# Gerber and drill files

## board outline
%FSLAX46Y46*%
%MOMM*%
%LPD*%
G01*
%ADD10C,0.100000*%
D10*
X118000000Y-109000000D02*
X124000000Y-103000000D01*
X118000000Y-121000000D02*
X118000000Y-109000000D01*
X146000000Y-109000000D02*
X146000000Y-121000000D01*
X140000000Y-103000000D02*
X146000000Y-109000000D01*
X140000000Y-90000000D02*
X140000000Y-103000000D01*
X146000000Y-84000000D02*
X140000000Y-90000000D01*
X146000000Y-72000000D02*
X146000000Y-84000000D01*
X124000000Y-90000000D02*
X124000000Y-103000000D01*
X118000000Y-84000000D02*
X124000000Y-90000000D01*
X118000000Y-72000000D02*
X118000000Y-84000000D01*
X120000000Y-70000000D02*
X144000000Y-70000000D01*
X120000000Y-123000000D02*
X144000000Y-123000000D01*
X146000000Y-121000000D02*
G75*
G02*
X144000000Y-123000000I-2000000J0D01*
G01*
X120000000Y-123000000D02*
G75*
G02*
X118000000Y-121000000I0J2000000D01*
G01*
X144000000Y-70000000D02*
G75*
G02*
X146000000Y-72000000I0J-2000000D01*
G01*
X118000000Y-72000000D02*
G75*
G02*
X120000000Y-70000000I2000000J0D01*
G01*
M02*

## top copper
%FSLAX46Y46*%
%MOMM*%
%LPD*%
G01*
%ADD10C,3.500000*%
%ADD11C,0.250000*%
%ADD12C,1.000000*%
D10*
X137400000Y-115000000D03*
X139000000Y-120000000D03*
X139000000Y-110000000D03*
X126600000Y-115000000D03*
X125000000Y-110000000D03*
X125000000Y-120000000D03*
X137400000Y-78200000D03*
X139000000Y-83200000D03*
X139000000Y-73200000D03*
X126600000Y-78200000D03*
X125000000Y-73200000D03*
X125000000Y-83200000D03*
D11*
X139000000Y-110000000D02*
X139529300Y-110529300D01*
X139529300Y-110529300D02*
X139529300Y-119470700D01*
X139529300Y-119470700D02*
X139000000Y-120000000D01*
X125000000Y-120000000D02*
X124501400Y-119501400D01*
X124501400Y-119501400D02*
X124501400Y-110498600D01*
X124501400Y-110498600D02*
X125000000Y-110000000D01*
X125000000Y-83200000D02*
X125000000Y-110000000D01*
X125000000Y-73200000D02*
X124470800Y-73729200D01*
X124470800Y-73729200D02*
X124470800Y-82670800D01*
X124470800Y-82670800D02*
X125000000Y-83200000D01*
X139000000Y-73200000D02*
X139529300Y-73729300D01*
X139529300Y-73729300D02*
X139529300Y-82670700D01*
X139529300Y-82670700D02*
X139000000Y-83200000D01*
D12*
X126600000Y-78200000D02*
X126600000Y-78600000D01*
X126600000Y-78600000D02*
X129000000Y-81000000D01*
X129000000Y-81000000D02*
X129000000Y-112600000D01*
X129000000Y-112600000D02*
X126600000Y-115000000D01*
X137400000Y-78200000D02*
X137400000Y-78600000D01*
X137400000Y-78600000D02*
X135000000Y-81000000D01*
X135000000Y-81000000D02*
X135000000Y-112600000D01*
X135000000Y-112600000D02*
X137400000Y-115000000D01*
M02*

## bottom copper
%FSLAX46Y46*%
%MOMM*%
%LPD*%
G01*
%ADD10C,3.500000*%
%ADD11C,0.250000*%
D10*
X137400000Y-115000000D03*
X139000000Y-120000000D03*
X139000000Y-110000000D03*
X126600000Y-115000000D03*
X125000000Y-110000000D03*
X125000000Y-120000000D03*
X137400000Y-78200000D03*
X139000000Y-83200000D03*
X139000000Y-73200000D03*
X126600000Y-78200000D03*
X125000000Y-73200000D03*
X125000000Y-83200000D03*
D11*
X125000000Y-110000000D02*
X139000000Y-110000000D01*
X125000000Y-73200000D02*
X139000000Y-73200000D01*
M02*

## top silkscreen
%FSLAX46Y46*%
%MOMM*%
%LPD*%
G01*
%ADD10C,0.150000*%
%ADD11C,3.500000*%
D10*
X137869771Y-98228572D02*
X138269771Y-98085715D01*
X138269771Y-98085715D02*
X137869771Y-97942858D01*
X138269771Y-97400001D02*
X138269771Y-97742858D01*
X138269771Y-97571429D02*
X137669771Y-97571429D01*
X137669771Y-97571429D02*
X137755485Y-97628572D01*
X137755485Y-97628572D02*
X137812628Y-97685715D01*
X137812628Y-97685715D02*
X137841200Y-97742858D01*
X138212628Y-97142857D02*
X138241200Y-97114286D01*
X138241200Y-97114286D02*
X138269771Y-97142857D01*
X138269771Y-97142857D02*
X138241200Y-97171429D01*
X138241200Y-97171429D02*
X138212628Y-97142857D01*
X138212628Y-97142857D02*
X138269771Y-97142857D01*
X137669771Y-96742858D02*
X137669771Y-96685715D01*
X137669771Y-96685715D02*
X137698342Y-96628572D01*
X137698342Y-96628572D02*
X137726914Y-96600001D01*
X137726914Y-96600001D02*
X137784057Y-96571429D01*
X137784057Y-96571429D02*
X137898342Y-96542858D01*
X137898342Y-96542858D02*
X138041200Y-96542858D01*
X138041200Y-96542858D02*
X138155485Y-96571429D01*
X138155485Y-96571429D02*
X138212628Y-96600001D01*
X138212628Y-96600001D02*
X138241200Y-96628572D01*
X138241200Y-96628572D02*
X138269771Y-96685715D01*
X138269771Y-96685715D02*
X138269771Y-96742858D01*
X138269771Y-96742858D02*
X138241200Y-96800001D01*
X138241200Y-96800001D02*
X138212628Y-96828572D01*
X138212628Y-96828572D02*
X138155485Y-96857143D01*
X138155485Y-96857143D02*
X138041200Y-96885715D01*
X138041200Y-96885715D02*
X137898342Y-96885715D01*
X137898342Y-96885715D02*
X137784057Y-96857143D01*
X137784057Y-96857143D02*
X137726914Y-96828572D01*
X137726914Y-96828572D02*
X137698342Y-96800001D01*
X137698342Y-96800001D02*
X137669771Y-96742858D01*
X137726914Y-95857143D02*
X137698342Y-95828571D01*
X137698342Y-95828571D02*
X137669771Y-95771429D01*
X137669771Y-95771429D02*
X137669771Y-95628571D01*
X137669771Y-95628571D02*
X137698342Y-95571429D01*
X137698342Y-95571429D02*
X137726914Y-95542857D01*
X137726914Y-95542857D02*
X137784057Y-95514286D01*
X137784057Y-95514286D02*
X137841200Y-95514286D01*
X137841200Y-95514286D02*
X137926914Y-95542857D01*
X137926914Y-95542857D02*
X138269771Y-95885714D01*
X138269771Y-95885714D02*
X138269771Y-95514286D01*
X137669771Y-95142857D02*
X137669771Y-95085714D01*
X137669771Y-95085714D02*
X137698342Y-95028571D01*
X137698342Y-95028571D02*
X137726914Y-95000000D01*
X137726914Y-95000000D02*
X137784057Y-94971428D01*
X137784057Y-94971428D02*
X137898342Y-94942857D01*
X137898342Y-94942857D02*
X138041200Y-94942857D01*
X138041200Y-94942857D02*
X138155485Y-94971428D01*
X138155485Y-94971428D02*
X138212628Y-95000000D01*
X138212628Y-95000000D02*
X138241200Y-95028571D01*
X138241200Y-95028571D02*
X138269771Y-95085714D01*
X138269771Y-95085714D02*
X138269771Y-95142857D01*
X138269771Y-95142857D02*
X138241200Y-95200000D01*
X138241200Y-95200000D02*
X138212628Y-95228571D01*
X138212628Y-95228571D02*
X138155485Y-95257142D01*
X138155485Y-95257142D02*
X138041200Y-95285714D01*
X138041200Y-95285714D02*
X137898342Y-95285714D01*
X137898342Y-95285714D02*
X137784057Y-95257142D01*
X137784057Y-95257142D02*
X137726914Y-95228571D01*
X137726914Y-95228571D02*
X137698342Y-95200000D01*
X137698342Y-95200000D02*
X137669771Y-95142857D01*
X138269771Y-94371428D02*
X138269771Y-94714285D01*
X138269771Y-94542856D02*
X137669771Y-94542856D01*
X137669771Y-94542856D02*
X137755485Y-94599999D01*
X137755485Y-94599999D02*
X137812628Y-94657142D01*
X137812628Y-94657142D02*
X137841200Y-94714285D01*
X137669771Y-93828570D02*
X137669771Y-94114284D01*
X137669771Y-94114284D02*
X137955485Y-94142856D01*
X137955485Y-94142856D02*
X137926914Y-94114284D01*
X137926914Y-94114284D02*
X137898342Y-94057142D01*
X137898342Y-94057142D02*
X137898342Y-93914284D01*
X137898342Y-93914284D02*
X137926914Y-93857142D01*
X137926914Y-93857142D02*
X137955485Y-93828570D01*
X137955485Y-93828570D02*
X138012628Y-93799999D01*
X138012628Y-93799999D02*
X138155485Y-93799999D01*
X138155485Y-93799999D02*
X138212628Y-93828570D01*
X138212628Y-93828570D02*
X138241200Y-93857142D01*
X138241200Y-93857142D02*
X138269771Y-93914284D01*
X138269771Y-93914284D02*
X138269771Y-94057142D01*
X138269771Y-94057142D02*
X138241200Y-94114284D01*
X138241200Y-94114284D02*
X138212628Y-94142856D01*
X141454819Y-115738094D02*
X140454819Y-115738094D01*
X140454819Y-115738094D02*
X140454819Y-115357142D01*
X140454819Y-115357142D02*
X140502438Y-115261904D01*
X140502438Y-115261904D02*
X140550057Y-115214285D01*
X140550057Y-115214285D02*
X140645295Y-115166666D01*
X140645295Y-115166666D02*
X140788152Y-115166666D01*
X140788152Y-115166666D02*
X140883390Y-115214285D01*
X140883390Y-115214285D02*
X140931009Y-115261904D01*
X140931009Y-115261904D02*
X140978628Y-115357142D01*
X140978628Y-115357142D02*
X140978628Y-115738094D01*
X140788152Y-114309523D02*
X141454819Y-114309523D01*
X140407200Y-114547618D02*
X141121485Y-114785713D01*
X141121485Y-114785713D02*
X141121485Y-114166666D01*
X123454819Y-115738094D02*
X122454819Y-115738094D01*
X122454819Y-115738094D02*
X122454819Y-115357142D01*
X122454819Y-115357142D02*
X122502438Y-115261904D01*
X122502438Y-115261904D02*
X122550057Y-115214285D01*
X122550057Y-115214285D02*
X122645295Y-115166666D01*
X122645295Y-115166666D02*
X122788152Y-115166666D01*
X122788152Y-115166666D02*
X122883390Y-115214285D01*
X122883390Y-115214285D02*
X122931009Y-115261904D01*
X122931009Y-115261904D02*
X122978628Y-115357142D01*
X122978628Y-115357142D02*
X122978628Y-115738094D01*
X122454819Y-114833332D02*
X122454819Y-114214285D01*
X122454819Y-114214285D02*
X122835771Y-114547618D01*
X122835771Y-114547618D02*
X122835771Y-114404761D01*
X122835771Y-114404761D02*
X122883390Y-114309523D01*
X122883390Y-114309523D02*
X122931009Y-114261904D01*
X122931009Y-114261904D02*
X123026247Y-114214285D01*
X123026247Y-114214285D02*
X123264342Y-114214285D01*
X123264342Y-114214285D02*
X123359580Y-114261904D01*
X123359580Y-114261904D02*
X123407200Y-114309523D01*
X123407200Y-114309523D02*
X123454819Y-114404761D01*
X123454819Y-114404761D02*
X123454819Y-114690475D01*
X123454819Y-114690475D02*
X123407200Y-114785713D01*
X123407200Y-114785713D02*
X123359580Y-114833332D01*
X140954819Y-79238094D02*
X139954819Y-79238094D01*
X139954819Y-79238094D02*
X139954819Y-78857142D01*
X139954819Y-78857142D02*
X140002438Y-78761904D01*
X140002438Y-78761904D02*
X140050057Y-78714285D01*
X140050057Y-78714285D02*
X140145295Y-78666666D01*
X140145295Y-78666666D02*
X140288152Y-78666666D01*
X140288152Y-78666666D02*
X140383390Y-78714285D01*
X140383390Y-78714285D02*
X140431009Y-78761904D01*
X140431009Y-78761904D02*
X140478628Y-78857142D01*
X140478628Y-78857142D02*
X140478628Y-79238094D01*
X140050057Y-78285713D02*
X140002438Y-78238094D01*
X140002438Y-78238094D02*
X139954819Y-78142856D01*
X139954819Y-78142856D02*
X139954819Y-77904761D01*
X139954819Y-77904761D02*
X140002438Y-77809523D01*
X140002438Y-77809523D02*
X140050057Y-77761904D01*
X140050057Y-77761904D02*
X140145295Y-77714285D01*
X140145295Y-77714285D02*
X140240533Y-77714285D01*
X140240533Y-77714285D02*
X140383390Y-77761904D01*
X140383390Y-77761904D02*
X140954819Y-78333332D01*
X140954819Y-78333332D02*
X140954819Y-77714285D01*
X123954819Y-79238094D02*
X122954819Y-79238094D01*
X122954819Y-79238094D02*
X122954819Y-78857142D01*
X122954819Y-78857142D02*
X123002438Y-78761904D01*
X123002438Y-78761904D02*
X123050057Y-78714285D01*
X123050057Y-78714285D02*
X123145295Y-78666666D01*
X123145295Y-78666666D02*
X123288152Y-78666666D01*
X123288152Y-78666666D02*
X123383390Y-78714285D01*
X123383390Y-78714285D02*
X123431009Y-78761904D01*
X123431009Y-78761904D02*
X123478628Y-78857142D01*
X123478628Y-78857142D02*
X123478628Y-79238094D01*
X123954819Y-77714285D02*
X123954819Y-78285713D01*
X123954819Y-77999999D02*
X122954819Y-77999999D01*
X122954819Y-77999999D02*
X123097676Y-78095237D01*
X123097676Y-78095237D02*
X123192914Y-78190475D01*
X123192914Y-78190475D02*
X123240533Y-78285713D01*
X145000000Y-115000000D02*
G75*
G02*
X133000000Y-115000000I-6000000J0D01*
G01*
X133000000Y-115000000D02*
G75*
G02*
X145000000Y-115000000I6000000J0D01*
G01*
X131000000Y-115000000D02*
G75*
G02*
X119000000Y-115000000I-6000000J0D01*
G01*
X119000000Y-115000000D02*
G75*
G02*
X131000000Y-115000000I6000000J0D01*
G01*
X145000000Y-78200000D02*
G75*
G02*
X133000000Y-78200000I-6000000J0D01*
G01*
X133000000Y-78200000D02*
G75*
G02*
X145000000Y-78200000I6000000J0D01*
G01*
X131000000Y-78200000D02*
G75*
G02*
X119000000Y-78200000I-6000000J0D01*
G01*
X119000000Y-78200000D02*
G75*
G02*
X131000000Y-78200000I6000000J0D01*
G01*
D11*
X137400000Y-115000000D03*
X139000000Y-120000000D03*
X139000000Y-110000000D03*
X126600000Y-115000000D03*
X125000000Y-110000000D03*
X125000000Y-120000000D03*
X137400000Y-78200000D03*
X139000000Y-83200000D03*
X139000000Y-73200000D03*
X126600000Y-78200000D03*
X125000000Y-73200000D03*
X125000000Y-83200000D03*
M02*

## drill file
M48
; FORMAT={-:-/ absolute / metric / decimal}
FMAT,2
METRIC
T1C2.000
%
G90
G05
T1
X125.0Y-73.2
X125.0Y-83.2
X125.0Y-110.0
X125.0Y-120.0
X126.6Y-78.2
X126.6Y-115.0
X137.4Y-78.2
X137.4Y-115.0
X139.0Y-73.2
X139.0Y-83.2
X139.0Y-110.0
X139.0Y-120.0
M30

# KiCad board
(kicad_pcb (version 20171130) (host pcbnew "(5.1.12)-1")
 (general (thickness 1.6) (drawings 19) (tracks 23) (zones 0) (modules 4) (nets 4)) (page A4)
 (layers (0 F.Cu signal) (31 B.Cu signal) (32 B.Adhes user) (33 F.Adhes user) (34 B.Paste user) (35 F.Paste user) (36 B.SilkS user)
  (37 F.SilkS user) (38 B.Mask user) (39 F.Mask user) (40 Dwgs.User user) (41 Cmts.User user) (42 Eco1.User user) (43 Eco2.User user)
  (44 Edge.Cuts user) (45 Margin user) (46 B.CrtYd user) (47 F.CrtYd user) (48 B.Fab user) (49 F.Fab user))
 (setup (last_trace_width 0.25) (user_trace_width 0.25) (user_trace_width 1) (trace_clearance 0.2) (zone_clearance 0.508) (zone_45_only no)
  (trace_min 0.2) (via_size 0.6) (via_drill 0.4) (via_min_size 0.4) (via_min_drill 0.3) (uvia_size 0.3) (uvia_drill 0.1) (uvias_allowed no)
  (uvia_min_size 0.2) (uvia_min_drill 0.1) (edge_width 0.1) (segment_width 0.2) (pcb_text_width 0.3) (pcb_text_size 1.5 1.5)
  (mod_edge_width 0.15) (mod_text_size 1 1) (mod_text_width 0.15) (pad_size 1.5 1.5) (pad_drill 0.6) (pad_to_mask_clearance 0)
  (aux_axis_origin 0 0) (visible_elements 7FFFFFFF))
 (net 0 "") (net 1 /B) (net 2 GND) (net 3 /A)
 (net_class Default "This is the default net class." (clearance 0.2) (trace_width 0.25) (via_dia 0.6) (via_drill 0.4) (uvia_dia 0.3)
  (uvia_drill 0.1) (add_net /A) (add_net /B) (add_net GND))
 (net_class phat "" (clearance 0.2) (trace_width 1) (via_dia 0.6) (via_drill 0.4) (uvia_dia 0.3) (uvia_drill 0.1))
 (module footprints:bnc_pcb (layer F.Cu) (at 139 115 90)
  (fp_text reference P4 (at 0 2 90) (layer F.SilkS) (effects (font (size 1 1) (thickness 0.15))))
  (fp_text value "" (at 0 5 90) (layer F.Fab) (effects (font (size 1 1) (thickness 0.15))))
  (fp_circle (center 0 0) (end 6 0) (layer F.SilkS) (width 0.15))
  (pad 1 thru_hole circle (at 0 -1.6 90) (size 3.5 3.5) (drill 2) (layers *.Cu *.Mask F.SilkS) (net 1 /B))
  (pad 2 thru_hole circle (at -5 0 90) (size 3.5 3.5) (drill 2) (layers *.Cu *.Mask F.SilkS) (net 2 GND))
  (pad 2 thru_hole circle (at 5 0 90) (size 3.5 3.5) (drill 2) (layers *.Cu *.Mask F.SilkS) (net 2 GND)))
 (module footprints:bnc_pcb (layer F.Cu) (at 125 115 270)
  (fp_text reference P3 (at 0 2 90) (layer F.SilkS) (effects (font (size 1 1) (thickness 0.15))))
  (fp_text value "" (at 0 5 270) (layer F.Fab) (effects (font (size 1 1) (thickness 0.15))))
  (fp_circle (center 0 0) (end 6 0) (layer F.SilkS) (width 0.15))
  (pad 1 thru_hole circle (at 0 -1.6 270) (size 3.5 3.5) (drill 2) (layers *.Cu *.Mask F.SilkS) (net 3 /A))
  (pad 2 thru_hole circle (at -5 0 270) (size 3.5 3.5) (drill 2) (layers *.Cu *.Mask F.SilkS) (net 2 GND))
  (pad 2 thru_hole circle (at 5 0 270) (size 3.5 3.5) (drill 2) (layers *.Cu *.Mask F.SilkS) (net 2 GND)))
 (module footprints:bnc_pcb (layer F.Cu) (at 139 78.2 90)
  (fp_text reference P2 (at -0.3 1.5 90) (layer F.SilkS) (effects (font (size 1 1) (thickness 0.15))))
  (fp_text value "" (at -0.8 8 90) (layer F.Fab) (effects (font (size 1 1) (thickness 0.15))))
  (fp_circle (center 0 0) (end 6 0) (layer F.SilkS) (width 0.15))
  (pad 1 thru_hole circle (at 0 -1.6 90) (size 3.5 3.5) (drill 2) (layers *.Cu *.Mask F.SilkS) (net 1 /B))
  (pad 2 thru_hole circle (at -5 0 90) (size 3.5 3.5) (drill 2) (layers *.Cu *.Mask F.SilkS) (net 2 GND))
  (pad 2 thru_hole circle (at 5 0 90) (size 3.5 3.5) (drill 2) (layers *.Cu *.Mask F.SilkS) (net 2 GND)))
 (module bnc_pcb (layer F.Cu) (at 125 78.2 270)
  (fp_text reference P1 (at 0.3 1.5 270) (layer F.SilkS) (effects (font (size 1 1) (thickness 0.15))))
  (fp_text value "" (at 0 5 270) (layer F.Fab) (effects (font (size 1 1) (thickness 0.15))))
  (fp_circle (center 0 0) (end 6 0) (layer F.SilkS) (width 0.15))
  (pad 1 thru_hole circle (at 0 -1.6 270) (size 3.5 3.5) (drill 2) (layers *.Cu *.Mask F.SilkS) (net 3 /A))
  (pad 2 thru_hole circle (at -5 0 270) (size 3.5 3.5) (drill 2) (layers *.Cu *.Mask F.SilkS) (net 2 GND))
  (pad 2 thru_hole circle (at 5 0 270) (size 3.5 3.5) (drill 2) (layers *.Cu *.Mask F.SilkS) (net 2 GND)))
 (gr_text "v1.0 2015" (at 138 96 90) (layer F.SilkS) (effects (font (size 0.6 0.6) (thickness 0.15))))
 (gr_line (start 118 109) (end 124 103) (angle 90) (layer Edge.Cuts) (width 0.1))
 (gr_line (start 118 121) (end 118 109) (angle 90) (layer Edge.Cuts) (width 0.1))
 (gr_line (start 146 109) (end 146 121) (angle 90) (layer Edge.Cuts) (width 0.1))
 (gr_line (start 140 103) (end 146 109) (angle 90) (layer Edge.Cuts) (width 0.1))
 (gr_line (start 140 90) (end 140 103) (angle 90) (layer Edge.Cuts) (width 0.1))
 (gr_line (start 146 84) (end 140 90) (angle 90) (layer Edge.Cuts) (width 0.1))
 (gr_line (start 146 72) (end 146 84) (angle 90) (layer Edge.Cuts) (width 0.1))
 (gr_line (start 124 90) (end 124 103) (angle 90) (layer Edge.Cuts) (width 0.1))
 (gr_line (start 118 84) (end 124 90) (angle 90) (layer Edge.Cuts) (width 0.1))
 (gr_line (start 118 72) (end 118 84) (angle 90) (layer Edge.Cuts) (width 0.1))
 (gr_line (start 120 70) (end 144 70) (angle 90) (layer Edge.Cuts) (width 0.1))
 (gr_line (start 120 123) (end 144 123) (angle 90) (layer Edge.Cuts) (width 0.1))
 (gr_arc (start 144 121) (end 146 121) (angle 90) (layer Edge.Cuts) (width 0.1))
 (gr_arc (start 120 121) (end 120 123) (angle 90) (layer Edge.Cuts) (width 0.1))
 (gr_arc (start 144 72) (end 144 70) (angle 90) (layer Edge.Cuts) (width 0.1))
 (gr_arc (start 120 72) (end 118 72) (angle 90) (layer Edge.Cuts) (width 0.1))
 (segment (start 139 110) (end 139.5293 110.5293) (width 0.25) (layer F.Cu) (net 2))
 (segment (start 139.5293 110.5293) (end 139.5293 119.4707) (width 0.25) (layer F.Cu) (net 2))
 (segment (start 139.5293 119.4707) (end 139 120) (width 0.25) (layer F.Cu) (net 2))
 (segment (start 125 110) (end 139 110) (width 0.25) (layer B.Cu) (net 2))
 (segment (start 125 120) (end 124.5014 119.5014) (width 0.25) (layer F.Cu) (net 2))
 (segment (start 124.5014 119.5014) (end 124.5014 110.4986) (width 0.25) (layer F.Cu) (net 2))
 (segment (start 124.5014 110.4986) (end 125 110) (width 0.25) (layer F.Cu) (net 2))
 (segment (start 125 83.2) (end 125 110) (width 0.25) (layer F.Cu) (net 2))
 (segment (start 125 73.2) (end 124.4708 73.7292) (width 0.25) (layer F.Cu) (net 2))
 (segment (start 124.4708 73.7292) (end 124.4708 82.6708) (width 0.25) (layer F.Cu) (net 2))
 (segment (start 124.4708 82.6708) (end 125 83.2) (width 0.25) (layer F.Cu) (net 2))
 (segment (start 139 73.2) (end 139.5293 73.7293) (width 0.25) (layer F.Cu) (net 2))
 (segment (start 139.5293 73.7293) (end 139.5293 82.6707) (width 0.25) (layer F.Cu) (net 2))
 (segment (start 139.5293 82.6707) (end 139 83.2) (width 0.25) (layer F.Cu) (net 2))
 (segment (start 125 73.2) (end 139 73.2) (width 0.25) (layer B.Cu) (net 2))
 (segment (start 126.6 78.2) (end 126.6 78.6) (width 1) (layer F.Cu) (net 3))
 (segment (start 126.6 78.6) (end 129 81) (width 1) (layer F.Cu) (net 3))
 (segment (start 129 81) (end 129 112.6) (width 1) (layer F.Cu) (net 3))
 (segment (start 129 112.6) (end 126.6 115) (width 1) (layer F.Cu) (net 3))
 (segment (start 137.4 78.2) (end 137.4 78.6) (width 1) (layer F.Cu) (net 1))
 (segment (start 137.4 78.6) (end 135 81) (width 1) (layer F.Cu) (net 1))
 (segment (start 135 81) (end 135 112.6) (width 1) (layer F.Cu) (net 1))
 (segment (start 135 112.6) (end 137.4 115) (width 1) (layer F.Cu) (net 1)))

